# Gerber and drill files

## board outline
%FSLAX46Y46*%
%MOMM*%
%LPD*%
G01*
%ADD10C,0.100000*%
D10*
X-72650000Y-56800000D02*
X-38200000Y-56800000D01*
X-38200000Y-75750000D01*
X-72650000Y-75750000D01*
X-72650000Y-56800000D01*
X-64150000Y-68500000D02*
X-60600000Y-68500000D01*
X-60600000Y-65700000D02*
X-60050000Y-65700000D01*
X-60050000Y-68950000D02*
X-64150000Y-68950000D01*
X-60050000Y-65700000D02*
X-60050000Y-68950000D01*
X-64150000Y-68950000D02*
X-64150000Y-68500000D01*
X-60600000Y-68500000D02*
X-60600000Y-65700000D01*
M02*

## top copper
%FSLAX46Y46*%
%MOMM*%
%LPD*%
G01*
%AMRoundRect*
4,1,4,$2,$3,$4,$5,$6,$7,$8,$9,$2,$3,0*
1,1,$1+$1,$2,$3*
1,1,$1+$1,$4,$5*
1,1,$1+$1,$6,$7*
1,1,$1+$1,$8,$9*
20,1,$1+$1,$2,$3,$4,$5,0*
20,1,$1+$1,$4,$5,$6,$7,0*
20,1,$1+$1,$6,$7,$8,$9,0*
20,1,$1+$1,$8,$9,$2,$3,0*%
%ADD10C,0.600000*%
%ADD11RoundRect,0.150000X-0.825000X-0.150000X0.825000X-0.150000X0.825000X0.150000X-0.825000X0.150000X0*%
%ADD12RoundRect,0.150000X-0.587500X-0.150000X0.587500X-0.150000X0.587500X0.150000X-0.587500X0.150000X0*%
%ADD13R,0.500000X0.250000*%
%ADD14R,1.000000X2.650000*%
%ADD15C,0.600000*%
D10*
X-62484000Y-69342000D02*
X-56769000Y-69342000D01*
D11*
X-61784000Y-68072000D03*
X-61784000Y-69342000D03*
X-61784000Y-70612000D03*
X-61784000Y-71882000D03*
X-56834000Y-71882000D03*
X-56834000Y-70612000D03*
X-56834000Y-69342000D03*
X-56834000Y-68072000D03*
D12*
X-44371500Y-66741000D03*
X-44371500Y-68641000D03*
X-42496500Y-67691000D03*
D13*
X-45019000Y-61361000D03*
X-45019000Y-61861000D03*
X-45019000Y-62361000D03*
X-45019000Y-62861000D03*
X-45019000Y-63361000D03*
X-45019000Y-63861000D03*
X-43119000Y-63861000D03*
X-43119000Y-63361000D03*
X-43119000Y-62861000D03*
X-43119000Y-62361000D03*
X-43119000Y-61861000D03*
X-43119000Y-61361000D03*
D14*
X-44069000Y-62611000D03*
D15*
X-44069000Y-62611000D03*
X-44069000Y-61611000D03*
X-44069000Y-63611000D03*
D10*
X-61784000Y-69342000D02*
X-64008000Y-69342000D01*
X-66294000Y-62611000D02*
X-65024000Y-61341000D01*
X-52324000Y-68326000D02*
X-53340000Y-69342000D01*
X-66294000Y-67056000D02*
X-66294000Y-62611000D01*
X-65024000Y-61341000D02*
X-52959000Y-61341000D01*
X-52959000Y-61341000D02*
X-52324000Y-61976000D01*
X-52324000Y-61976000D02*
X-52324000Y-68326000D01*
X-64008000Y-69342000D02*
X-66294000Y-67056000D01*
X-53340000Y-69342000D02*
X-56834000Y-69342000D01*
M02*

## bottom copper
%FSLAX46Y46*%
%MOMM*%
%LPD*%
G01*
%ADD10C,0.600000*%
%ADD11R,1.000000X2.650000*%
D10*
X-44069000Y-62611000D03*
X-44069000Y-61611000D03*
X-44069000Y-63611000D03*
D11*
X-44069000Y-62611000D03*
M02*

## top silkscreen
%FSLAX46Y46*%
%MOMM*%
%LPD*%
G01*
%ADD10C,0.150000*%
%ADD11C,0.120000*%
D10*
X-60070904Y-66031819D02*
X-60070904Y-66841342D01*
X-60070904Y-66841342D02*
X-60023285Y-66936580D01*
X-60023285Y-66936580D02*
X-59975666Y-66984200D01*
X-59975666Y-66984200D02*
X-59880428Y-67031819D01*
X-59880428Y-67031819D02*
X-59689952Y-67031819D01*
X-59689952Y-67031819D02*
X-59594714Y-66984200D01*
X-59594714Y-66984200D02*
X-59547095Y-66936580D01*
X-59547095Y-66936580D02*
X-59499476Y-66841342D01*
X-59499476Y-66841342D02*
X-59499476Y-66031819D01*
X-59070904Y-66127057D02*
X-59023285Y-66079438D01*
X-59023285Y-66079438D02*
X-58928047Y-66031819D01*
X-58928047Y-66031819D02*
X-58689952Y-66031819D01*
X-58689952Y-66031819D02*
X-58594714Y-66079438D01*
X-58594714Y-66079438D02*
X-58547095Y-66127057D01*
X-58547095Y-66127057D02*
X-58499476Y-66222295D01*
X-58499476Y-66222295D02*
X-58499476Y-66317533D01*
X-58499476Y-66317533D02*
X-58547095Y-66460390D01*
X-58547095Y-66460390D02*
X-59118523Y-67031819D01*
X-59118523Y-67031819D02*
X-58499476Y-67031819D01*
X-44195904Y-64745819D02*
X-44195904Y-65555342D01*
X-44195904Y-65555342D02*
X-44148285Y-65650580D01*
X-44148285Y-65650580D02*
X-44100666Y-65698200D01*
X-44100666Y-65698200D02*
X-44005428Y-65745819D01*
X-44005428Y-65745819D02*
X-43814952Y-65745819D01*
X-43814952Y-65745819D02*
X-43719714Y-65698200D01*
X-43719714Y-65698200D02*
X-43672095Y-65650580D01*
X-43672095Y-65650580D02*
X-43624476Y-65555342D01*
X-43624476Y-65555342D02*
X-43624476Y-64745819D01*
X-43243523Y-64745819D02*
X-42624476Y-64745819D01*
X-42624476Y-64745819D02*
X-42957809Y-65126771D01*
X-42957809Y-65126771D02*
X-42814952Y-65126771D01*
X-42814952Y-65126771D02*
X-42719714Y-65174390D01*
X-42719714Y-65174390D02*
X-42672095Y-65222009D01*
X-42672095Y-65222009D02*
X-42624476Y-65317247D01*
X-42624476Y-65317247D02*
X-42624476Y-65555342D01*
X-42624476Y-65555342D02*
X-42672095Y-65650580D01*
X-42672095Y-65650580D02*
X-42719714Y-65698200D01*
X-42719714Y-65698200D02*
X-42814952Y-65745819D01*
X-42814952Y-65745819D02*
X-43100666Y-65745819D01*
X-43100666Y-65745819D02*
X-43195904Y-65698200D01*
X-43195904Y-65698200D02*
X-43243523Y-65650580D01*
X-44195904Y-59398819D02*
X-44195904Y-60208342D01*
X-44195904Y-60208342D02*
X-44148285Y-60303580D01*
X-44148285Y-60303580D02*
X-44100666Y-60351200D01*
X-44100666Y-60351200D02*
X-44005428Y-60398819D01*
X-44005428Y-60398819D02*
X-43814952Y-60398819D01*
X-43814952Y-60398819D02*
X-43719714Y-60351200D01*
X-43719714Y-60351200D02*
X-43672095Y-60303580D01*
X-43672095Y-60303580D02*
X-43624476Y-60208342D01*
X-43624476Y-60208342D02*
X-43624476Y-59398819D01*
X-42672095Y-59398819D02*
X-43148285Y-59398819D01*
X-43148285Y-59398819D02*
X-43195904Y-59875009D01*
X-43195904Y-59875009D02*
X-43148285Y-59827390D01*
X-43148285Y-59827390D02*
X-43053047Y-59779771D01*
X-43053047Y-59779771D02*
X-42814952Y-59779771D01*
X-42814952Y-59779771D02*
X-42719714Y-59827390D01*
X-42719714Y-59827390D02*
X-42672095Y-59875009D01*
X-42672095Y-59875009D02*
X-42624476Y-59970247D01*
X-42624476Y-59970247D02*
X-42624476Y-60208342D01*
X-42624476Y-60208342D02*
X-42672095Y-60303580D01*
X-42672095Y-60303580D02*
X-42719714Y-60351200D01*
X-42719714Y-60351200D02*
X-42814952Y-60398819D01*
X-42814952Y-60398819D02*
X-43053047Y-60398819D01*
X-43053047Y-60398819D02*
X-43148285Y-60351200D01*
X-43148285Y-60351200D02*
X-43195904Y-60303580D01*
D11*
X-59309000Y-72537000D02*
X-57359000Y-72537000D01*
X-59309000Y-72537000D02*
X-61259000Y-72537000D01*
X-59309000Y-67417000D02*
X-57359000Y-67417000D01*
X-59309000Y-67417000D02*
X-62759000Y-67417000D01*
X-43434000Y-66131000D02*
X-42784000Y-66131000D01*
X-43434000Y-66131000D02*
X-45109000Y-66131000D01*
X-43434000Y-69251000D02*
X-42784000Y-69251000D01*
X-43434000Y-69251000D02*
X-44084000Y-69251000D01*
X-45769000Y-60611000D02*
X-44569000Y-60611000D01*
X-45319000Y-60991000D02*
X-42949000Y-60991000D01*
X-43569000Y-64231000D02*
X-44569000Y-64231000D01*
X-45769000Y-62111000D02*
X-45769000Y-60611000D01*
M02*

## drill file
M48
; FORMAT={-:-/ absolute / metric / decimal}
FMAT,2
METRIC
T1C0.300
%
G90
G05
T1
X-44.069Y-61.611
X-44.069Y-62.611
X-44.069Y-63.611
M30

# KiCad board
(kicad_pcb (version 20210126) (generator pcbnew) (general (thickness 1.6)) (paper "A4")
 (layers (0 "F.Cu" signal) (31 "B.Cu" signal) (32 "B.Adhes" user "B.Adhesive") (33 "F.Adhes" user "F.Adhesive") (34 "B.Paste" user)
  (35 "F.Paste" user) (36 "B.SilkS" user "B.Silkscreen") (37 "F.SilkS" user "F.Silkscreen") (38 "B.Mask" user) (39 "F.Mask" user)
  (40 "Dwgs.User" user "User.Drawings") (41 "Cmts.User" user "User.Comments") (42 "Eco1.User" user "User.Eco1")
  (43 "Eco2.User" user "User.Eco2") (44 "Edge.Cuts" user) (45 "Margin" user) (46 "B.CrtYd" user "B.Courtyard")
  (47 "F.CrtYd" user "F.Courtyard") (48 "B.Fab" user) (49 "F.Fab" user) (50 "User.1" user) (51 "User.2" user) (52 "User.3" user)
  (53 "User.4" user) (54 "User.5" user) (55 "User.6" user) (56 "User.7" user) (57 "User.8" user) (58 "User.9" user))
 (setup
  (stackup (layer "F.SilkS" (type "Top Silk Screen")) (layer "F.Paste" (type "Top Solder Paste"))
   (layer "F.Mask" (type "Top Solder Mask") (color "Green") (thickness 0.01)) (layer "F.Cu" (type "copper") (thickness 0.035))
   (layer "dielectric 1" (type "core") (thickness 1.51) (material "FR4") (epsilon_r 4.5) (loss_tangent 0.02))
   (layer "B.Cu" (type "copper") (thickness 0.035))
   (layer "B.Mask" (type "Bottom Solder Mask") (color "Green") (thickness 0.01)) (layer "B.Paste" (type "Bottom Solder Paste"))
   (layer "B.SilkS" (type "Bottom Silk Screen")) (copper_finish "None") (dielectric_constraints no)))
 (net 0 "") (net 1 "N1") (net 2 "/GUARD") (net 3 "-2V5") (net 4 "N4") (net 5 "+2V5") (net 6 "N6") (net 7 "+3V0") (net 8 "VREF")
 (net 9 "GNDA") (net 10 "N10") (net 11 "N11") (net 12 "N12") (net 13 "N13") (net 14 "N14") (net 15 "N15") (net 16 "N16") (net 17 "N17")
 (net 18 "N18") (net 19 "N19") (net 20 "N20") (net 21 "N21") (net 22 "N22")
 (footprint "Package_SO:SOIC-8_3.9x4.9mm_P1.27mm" (layer "F.Cu") (at -59.309 69.977)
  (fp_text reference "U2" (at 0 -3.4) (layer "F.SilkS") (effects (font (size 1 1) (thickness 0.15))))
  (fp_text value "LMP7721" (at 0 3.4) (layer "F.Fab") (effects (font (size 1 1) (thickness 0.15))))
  (fp_line (start 0 2.56) (end 1.95 2.56) (layer "F.SilkS") (width 0.12))
  (fp_line (start 0 2.56) (end -1.95 2.56) (layer "F.SilkS") (width 0.12))
  (fp_line (start 0 -2.56) (end 1.95 -2.56) (layer "F.SilkS") (width 0.12))
  (fp_line (start 0 -2.56) (end -3.45 -2.56) (layer "F.SilkS") (width 0.12))
  (pad "1" smd roundrect (at -2.475 -1.905) (locked) (size 1.95 0.6) (layers "F.Cu" "F.Paste" "F.Mask") (roundrect_rratio 0.25) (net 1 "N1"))
  (pad "2" smd roundrect (at -2.475 -0.635) (locked) (size 1.95 0.6) (layers "F.Cu" "F.Paste" "F.Mask") (roundrect_rratio 0.25)
   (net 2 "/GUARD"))
  (pad "3" smd roundrect (at -2.475 0.635) (locked) (size 1.95 0.6) (layers "F.Cu" "F.Paste" "F.Mask") (roundrect_rratio 0.25)
   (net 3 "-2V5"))
  (pad "4" smd roundrect (at -2.475 1.905) (locked) (size 1.95 0.6) (layers "F.Cu" "F.Paste" "F.Mask") (roundrect_rratio 0.25) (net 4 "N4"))
  (pad "5" smd roundrect (at 2.475 1.905) (locked) (size 1.95 0.6) (layers "F.Cu" "F.Paste" "F.Mask") (roundrect_rratio 0.25))
  (pad "6" smd roundrect (at 2.475 0.635) (locked) (size 1.95 0.6) (layers "F.Cu" "F.Paste" "F.Mask") (roundrect_rratio 0.25) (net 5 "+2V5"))
  (pad "7" smd roundrect (at 2.475 -0.635) (locked) (size 1.95 0.6) (layers "F.Cu" "F.Paste" "F.Mask") (roundrect_rratio 0.25)
   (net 2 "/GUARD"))
  (pad "8" smd roundrect (at 2.475 -1.905) (locked) (size 1.95 0.6) (layers "F.Cu" "F.Paste" "F.Mask") (roundrect_rratio 0.25) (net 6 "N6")))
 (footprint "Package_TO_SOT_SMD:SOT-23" (layer "F.Cu") (at -43.434 67.691)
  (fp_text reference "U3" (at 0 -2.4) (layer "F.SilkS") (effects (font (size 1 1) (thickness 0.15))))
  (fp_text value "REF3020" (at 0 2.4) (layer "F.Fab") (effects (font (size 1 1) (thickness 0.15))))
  (fp_line (start 0 -1.56) (end 0.65 -1.56) (layer "F.SilkS") (width 0.12))
  (fp_line (start 0 -1.56) (end -1.675 -1.56) (layer "F.SilkS") (width 0.12))
  (fp_line (start 0 1.56) (end 0.65 1.56) (layer "F.SilkS") (width 0.12))
  (fp_line (start 0 1.56) (end -0.65 1.56) (layer "F.SilkS") (width 0.12))
  (pad "1" smd roundrect (at -0.9375 -0.95) (locked) (size 1.475 0.6) (layers "F.Cu" "F.Paste" "F.Mask") (roundrect_rratio 0.25)
   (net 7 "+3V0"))
  (pad "2" smd roundrect (at -0.9375 0.95) (locked) (size 1.475 0.6) (layers "F.Cu" "F.Paste" "F.Mask") (roundrect_rratio 0.25)
   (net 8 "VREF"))
  (pad "3" smd roundrect (at 0.9375 0) (locked) (size 1.475 0.6) (layers "F.Cu" "F.Paste" "F.Mask") (roundrect_rratio 0.25) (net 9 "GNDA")))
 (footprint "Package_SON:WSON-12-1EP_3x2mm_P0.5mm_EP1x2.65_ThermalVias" (layer "F.Cu") (at -44.069 62.611)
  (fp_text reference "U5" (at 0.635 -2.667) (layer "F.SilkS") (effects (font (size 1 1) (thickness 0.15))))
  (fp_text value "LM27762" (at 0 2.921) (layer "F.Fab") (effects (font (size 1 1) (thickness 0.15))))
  (fp_line (start -1.7 -2) (end -0.5 -2) (layer "F.SilkS") (width 0.12))
  (fp_line (start -1.25 -1.62) (end 1.12 -1.62) (layer "F.SilkS") (width 0.12))
  (fp_line (start 0.5 1.62) (end -0.5 1.62) (layer "F.SilkS") (width 0.12))
  (fp_line (start -1.7 -0.5) (end -1.7 -2) (layer "F.SilkS") (width 0.12))
  (pad "" smd rect (at 0 0.5) (locked) (size 0.95 0.8) (layers "F.Paste"))
  (pad "" smd rect (at 0 -0.5) (locked) (size 0.95 0.8) (layers "F.Paste"))
  (pad "1" smd rect (at -0.95 -1.25) (locked) (size 0.5 0.25) (layers "F.Cu" "F.Paste" "F.Mask") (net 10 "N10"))
  (pad "2" smd rect (at -0.95 -0.75) (locked) (size 0.5 0.25) (layers "F.Cu" "F.Paste" "F.Mask") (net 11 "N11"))
  (pad "3" smd rect (at -0.95 -0.25) (locked) (size 0.5 0.25) (layers "F.Cu" "F.Paste" "F.Mask") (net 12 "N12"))
  (pad "4" smd rect (at -0.95 0.25) (locked) (size 0.5 0.25) (layers "F.Cu" "F.Paste" "F.Mask") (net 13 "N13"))
  (pad "5" smd rect (at -0.95 0.75) (locked) (size 0.5 0.25) (layers "F.Cu" "F.Paste" "F.Mask") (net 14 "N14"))
  (pad "6" smd rect (at -0.95 1.25) (locked) (size 0.5 0.25) (layers "F.Cu" "F.Paste" "F.Mask") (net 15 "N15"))
  (pad "7" smd rect (at 0.95 1.25) (locked) (size 0.5 0.25) (layers "F.Cu" "F.Paste" "F.Mask") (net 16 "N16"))
  (pad "8" smd rect (at 0.95 0.75) (locked) (size 0.5 0.25) (layers "F.Cu" "F.Paste" "F.Mask") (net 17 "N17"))
  (pad "9" smd rect (at 0.95 0.25) (locked) (size 0.5 0.25) (layers "F.Cu" "F.Paste" "F.Mask") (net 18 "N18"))
  (pad "10" smd rect (at 0.95 -0.25) (locked) (size 0.5 0.25) (layers "F.Cu" "F.Paste" "F.Mask") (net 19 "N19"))
  (pad "11" smd rect (at 0.95 -0.75) (locked) (size 0.5 0.25) (layers "F.Cu" "F.Paste" "F.Mask") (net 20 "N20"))
  (pad "12" smd rect (at 0.95 -1.25) (locked) (size 0.5 0.25) (layers "F.Cu" "F.Paste" "F.Mask") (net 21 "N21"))
  (pad "13" smd rect (at 0 0) (locked) (size 1 2.65) (layers "F.Cu" "F.Mask") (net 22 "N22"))
  (pad "13" thru_hole circle (at 0 0) (locked) (size 0.6 0.6) (drill 0.3) (layers *.Cu) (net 22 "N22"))
  (pad "13" thru_hole circle (at 0 -1 90) (locked) (size 0.6 0.6) (drill 0.3) (layers *.Cu) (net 22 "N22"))
  (pad "13" thru_hole circle (at 0 1) (locked) (size 0.6 0.6) (drill 0.3) (layers *.Cu) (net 22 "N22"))
  (pad "13" smd rect (at 0 0) (locked) (size 1 2.65) (layers "B.Cu") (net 22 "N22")))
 (gr_line (start -62.484 69.342) (end -56.769 69.342) (layer "F.Cu") (width 0.6))
 (gr_rect (start -72.65 56.8) (end -38.2 75.75) (layer "Edge.Cuts") (width 0.1) (fill none))
 (gr_line (start -64.15 68.5) (end -60.6 68.5) (layer "Edge.Cuts") (width 0.1))
 (gr_line (start -60.6 65.7) (end -60.05 65.7) (layer "Edge.Cuts") (width 0.1))
 (gr_line (start -60.05 68.95) (end -64.15 68.95) (layer "Edge.Cuts") (width 0.1))
 (gr_line (start -60.05 65.7) (end -60.05 68.95) (layer "Edge.Cuts") (width 0.1))
 (gr_line (start -64.15 68.95) (end -64.15 68.5) (layer "Edge.Cuts") (width 0.1))
 (gr_line (start -60.6 68.5) (end -60.6 65.7) (layer "Edge.Cuts") (width 0.1))
 (segment (start -61.784 69.342) (end -64.008 69.342) (width 0.6) (layer "F.Cu") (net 2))
 (segment (start -66.294 62.611) (end -65.024 61.341) (width 0.6) (layer "F.Cu") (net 2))
 (segment (start -52.324 68.326) (end -53.34 69.342) (width 0.6) (layer "F.Cu") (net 2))
 (segment (start -66.294 67.056) (end -66.294 62.611) (width 0.6) (layer "F.Cu") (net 2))
 (segment (start -65.024 61.341) (end -52.959 61.341) (width 0.6) (layer "F.Cu") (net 2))
 (segment (start -52.959 61.341) (end -52.324 61.976) (width 0.6) (layer "F.Cu") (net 2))
 (segment (start -52.324 61.976) (end -52.324 68.326) (width 0.6) (layer "F.Cu") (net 2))
 (segment (start -64.008 69.342) (end -66.294 67.056) (width 0.6) (layer "F.Cu") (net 2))
 (segment (start -53.34 69.342) (end -56.834 69.342) (width 0.6) (layer "F.Cu") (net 2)))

